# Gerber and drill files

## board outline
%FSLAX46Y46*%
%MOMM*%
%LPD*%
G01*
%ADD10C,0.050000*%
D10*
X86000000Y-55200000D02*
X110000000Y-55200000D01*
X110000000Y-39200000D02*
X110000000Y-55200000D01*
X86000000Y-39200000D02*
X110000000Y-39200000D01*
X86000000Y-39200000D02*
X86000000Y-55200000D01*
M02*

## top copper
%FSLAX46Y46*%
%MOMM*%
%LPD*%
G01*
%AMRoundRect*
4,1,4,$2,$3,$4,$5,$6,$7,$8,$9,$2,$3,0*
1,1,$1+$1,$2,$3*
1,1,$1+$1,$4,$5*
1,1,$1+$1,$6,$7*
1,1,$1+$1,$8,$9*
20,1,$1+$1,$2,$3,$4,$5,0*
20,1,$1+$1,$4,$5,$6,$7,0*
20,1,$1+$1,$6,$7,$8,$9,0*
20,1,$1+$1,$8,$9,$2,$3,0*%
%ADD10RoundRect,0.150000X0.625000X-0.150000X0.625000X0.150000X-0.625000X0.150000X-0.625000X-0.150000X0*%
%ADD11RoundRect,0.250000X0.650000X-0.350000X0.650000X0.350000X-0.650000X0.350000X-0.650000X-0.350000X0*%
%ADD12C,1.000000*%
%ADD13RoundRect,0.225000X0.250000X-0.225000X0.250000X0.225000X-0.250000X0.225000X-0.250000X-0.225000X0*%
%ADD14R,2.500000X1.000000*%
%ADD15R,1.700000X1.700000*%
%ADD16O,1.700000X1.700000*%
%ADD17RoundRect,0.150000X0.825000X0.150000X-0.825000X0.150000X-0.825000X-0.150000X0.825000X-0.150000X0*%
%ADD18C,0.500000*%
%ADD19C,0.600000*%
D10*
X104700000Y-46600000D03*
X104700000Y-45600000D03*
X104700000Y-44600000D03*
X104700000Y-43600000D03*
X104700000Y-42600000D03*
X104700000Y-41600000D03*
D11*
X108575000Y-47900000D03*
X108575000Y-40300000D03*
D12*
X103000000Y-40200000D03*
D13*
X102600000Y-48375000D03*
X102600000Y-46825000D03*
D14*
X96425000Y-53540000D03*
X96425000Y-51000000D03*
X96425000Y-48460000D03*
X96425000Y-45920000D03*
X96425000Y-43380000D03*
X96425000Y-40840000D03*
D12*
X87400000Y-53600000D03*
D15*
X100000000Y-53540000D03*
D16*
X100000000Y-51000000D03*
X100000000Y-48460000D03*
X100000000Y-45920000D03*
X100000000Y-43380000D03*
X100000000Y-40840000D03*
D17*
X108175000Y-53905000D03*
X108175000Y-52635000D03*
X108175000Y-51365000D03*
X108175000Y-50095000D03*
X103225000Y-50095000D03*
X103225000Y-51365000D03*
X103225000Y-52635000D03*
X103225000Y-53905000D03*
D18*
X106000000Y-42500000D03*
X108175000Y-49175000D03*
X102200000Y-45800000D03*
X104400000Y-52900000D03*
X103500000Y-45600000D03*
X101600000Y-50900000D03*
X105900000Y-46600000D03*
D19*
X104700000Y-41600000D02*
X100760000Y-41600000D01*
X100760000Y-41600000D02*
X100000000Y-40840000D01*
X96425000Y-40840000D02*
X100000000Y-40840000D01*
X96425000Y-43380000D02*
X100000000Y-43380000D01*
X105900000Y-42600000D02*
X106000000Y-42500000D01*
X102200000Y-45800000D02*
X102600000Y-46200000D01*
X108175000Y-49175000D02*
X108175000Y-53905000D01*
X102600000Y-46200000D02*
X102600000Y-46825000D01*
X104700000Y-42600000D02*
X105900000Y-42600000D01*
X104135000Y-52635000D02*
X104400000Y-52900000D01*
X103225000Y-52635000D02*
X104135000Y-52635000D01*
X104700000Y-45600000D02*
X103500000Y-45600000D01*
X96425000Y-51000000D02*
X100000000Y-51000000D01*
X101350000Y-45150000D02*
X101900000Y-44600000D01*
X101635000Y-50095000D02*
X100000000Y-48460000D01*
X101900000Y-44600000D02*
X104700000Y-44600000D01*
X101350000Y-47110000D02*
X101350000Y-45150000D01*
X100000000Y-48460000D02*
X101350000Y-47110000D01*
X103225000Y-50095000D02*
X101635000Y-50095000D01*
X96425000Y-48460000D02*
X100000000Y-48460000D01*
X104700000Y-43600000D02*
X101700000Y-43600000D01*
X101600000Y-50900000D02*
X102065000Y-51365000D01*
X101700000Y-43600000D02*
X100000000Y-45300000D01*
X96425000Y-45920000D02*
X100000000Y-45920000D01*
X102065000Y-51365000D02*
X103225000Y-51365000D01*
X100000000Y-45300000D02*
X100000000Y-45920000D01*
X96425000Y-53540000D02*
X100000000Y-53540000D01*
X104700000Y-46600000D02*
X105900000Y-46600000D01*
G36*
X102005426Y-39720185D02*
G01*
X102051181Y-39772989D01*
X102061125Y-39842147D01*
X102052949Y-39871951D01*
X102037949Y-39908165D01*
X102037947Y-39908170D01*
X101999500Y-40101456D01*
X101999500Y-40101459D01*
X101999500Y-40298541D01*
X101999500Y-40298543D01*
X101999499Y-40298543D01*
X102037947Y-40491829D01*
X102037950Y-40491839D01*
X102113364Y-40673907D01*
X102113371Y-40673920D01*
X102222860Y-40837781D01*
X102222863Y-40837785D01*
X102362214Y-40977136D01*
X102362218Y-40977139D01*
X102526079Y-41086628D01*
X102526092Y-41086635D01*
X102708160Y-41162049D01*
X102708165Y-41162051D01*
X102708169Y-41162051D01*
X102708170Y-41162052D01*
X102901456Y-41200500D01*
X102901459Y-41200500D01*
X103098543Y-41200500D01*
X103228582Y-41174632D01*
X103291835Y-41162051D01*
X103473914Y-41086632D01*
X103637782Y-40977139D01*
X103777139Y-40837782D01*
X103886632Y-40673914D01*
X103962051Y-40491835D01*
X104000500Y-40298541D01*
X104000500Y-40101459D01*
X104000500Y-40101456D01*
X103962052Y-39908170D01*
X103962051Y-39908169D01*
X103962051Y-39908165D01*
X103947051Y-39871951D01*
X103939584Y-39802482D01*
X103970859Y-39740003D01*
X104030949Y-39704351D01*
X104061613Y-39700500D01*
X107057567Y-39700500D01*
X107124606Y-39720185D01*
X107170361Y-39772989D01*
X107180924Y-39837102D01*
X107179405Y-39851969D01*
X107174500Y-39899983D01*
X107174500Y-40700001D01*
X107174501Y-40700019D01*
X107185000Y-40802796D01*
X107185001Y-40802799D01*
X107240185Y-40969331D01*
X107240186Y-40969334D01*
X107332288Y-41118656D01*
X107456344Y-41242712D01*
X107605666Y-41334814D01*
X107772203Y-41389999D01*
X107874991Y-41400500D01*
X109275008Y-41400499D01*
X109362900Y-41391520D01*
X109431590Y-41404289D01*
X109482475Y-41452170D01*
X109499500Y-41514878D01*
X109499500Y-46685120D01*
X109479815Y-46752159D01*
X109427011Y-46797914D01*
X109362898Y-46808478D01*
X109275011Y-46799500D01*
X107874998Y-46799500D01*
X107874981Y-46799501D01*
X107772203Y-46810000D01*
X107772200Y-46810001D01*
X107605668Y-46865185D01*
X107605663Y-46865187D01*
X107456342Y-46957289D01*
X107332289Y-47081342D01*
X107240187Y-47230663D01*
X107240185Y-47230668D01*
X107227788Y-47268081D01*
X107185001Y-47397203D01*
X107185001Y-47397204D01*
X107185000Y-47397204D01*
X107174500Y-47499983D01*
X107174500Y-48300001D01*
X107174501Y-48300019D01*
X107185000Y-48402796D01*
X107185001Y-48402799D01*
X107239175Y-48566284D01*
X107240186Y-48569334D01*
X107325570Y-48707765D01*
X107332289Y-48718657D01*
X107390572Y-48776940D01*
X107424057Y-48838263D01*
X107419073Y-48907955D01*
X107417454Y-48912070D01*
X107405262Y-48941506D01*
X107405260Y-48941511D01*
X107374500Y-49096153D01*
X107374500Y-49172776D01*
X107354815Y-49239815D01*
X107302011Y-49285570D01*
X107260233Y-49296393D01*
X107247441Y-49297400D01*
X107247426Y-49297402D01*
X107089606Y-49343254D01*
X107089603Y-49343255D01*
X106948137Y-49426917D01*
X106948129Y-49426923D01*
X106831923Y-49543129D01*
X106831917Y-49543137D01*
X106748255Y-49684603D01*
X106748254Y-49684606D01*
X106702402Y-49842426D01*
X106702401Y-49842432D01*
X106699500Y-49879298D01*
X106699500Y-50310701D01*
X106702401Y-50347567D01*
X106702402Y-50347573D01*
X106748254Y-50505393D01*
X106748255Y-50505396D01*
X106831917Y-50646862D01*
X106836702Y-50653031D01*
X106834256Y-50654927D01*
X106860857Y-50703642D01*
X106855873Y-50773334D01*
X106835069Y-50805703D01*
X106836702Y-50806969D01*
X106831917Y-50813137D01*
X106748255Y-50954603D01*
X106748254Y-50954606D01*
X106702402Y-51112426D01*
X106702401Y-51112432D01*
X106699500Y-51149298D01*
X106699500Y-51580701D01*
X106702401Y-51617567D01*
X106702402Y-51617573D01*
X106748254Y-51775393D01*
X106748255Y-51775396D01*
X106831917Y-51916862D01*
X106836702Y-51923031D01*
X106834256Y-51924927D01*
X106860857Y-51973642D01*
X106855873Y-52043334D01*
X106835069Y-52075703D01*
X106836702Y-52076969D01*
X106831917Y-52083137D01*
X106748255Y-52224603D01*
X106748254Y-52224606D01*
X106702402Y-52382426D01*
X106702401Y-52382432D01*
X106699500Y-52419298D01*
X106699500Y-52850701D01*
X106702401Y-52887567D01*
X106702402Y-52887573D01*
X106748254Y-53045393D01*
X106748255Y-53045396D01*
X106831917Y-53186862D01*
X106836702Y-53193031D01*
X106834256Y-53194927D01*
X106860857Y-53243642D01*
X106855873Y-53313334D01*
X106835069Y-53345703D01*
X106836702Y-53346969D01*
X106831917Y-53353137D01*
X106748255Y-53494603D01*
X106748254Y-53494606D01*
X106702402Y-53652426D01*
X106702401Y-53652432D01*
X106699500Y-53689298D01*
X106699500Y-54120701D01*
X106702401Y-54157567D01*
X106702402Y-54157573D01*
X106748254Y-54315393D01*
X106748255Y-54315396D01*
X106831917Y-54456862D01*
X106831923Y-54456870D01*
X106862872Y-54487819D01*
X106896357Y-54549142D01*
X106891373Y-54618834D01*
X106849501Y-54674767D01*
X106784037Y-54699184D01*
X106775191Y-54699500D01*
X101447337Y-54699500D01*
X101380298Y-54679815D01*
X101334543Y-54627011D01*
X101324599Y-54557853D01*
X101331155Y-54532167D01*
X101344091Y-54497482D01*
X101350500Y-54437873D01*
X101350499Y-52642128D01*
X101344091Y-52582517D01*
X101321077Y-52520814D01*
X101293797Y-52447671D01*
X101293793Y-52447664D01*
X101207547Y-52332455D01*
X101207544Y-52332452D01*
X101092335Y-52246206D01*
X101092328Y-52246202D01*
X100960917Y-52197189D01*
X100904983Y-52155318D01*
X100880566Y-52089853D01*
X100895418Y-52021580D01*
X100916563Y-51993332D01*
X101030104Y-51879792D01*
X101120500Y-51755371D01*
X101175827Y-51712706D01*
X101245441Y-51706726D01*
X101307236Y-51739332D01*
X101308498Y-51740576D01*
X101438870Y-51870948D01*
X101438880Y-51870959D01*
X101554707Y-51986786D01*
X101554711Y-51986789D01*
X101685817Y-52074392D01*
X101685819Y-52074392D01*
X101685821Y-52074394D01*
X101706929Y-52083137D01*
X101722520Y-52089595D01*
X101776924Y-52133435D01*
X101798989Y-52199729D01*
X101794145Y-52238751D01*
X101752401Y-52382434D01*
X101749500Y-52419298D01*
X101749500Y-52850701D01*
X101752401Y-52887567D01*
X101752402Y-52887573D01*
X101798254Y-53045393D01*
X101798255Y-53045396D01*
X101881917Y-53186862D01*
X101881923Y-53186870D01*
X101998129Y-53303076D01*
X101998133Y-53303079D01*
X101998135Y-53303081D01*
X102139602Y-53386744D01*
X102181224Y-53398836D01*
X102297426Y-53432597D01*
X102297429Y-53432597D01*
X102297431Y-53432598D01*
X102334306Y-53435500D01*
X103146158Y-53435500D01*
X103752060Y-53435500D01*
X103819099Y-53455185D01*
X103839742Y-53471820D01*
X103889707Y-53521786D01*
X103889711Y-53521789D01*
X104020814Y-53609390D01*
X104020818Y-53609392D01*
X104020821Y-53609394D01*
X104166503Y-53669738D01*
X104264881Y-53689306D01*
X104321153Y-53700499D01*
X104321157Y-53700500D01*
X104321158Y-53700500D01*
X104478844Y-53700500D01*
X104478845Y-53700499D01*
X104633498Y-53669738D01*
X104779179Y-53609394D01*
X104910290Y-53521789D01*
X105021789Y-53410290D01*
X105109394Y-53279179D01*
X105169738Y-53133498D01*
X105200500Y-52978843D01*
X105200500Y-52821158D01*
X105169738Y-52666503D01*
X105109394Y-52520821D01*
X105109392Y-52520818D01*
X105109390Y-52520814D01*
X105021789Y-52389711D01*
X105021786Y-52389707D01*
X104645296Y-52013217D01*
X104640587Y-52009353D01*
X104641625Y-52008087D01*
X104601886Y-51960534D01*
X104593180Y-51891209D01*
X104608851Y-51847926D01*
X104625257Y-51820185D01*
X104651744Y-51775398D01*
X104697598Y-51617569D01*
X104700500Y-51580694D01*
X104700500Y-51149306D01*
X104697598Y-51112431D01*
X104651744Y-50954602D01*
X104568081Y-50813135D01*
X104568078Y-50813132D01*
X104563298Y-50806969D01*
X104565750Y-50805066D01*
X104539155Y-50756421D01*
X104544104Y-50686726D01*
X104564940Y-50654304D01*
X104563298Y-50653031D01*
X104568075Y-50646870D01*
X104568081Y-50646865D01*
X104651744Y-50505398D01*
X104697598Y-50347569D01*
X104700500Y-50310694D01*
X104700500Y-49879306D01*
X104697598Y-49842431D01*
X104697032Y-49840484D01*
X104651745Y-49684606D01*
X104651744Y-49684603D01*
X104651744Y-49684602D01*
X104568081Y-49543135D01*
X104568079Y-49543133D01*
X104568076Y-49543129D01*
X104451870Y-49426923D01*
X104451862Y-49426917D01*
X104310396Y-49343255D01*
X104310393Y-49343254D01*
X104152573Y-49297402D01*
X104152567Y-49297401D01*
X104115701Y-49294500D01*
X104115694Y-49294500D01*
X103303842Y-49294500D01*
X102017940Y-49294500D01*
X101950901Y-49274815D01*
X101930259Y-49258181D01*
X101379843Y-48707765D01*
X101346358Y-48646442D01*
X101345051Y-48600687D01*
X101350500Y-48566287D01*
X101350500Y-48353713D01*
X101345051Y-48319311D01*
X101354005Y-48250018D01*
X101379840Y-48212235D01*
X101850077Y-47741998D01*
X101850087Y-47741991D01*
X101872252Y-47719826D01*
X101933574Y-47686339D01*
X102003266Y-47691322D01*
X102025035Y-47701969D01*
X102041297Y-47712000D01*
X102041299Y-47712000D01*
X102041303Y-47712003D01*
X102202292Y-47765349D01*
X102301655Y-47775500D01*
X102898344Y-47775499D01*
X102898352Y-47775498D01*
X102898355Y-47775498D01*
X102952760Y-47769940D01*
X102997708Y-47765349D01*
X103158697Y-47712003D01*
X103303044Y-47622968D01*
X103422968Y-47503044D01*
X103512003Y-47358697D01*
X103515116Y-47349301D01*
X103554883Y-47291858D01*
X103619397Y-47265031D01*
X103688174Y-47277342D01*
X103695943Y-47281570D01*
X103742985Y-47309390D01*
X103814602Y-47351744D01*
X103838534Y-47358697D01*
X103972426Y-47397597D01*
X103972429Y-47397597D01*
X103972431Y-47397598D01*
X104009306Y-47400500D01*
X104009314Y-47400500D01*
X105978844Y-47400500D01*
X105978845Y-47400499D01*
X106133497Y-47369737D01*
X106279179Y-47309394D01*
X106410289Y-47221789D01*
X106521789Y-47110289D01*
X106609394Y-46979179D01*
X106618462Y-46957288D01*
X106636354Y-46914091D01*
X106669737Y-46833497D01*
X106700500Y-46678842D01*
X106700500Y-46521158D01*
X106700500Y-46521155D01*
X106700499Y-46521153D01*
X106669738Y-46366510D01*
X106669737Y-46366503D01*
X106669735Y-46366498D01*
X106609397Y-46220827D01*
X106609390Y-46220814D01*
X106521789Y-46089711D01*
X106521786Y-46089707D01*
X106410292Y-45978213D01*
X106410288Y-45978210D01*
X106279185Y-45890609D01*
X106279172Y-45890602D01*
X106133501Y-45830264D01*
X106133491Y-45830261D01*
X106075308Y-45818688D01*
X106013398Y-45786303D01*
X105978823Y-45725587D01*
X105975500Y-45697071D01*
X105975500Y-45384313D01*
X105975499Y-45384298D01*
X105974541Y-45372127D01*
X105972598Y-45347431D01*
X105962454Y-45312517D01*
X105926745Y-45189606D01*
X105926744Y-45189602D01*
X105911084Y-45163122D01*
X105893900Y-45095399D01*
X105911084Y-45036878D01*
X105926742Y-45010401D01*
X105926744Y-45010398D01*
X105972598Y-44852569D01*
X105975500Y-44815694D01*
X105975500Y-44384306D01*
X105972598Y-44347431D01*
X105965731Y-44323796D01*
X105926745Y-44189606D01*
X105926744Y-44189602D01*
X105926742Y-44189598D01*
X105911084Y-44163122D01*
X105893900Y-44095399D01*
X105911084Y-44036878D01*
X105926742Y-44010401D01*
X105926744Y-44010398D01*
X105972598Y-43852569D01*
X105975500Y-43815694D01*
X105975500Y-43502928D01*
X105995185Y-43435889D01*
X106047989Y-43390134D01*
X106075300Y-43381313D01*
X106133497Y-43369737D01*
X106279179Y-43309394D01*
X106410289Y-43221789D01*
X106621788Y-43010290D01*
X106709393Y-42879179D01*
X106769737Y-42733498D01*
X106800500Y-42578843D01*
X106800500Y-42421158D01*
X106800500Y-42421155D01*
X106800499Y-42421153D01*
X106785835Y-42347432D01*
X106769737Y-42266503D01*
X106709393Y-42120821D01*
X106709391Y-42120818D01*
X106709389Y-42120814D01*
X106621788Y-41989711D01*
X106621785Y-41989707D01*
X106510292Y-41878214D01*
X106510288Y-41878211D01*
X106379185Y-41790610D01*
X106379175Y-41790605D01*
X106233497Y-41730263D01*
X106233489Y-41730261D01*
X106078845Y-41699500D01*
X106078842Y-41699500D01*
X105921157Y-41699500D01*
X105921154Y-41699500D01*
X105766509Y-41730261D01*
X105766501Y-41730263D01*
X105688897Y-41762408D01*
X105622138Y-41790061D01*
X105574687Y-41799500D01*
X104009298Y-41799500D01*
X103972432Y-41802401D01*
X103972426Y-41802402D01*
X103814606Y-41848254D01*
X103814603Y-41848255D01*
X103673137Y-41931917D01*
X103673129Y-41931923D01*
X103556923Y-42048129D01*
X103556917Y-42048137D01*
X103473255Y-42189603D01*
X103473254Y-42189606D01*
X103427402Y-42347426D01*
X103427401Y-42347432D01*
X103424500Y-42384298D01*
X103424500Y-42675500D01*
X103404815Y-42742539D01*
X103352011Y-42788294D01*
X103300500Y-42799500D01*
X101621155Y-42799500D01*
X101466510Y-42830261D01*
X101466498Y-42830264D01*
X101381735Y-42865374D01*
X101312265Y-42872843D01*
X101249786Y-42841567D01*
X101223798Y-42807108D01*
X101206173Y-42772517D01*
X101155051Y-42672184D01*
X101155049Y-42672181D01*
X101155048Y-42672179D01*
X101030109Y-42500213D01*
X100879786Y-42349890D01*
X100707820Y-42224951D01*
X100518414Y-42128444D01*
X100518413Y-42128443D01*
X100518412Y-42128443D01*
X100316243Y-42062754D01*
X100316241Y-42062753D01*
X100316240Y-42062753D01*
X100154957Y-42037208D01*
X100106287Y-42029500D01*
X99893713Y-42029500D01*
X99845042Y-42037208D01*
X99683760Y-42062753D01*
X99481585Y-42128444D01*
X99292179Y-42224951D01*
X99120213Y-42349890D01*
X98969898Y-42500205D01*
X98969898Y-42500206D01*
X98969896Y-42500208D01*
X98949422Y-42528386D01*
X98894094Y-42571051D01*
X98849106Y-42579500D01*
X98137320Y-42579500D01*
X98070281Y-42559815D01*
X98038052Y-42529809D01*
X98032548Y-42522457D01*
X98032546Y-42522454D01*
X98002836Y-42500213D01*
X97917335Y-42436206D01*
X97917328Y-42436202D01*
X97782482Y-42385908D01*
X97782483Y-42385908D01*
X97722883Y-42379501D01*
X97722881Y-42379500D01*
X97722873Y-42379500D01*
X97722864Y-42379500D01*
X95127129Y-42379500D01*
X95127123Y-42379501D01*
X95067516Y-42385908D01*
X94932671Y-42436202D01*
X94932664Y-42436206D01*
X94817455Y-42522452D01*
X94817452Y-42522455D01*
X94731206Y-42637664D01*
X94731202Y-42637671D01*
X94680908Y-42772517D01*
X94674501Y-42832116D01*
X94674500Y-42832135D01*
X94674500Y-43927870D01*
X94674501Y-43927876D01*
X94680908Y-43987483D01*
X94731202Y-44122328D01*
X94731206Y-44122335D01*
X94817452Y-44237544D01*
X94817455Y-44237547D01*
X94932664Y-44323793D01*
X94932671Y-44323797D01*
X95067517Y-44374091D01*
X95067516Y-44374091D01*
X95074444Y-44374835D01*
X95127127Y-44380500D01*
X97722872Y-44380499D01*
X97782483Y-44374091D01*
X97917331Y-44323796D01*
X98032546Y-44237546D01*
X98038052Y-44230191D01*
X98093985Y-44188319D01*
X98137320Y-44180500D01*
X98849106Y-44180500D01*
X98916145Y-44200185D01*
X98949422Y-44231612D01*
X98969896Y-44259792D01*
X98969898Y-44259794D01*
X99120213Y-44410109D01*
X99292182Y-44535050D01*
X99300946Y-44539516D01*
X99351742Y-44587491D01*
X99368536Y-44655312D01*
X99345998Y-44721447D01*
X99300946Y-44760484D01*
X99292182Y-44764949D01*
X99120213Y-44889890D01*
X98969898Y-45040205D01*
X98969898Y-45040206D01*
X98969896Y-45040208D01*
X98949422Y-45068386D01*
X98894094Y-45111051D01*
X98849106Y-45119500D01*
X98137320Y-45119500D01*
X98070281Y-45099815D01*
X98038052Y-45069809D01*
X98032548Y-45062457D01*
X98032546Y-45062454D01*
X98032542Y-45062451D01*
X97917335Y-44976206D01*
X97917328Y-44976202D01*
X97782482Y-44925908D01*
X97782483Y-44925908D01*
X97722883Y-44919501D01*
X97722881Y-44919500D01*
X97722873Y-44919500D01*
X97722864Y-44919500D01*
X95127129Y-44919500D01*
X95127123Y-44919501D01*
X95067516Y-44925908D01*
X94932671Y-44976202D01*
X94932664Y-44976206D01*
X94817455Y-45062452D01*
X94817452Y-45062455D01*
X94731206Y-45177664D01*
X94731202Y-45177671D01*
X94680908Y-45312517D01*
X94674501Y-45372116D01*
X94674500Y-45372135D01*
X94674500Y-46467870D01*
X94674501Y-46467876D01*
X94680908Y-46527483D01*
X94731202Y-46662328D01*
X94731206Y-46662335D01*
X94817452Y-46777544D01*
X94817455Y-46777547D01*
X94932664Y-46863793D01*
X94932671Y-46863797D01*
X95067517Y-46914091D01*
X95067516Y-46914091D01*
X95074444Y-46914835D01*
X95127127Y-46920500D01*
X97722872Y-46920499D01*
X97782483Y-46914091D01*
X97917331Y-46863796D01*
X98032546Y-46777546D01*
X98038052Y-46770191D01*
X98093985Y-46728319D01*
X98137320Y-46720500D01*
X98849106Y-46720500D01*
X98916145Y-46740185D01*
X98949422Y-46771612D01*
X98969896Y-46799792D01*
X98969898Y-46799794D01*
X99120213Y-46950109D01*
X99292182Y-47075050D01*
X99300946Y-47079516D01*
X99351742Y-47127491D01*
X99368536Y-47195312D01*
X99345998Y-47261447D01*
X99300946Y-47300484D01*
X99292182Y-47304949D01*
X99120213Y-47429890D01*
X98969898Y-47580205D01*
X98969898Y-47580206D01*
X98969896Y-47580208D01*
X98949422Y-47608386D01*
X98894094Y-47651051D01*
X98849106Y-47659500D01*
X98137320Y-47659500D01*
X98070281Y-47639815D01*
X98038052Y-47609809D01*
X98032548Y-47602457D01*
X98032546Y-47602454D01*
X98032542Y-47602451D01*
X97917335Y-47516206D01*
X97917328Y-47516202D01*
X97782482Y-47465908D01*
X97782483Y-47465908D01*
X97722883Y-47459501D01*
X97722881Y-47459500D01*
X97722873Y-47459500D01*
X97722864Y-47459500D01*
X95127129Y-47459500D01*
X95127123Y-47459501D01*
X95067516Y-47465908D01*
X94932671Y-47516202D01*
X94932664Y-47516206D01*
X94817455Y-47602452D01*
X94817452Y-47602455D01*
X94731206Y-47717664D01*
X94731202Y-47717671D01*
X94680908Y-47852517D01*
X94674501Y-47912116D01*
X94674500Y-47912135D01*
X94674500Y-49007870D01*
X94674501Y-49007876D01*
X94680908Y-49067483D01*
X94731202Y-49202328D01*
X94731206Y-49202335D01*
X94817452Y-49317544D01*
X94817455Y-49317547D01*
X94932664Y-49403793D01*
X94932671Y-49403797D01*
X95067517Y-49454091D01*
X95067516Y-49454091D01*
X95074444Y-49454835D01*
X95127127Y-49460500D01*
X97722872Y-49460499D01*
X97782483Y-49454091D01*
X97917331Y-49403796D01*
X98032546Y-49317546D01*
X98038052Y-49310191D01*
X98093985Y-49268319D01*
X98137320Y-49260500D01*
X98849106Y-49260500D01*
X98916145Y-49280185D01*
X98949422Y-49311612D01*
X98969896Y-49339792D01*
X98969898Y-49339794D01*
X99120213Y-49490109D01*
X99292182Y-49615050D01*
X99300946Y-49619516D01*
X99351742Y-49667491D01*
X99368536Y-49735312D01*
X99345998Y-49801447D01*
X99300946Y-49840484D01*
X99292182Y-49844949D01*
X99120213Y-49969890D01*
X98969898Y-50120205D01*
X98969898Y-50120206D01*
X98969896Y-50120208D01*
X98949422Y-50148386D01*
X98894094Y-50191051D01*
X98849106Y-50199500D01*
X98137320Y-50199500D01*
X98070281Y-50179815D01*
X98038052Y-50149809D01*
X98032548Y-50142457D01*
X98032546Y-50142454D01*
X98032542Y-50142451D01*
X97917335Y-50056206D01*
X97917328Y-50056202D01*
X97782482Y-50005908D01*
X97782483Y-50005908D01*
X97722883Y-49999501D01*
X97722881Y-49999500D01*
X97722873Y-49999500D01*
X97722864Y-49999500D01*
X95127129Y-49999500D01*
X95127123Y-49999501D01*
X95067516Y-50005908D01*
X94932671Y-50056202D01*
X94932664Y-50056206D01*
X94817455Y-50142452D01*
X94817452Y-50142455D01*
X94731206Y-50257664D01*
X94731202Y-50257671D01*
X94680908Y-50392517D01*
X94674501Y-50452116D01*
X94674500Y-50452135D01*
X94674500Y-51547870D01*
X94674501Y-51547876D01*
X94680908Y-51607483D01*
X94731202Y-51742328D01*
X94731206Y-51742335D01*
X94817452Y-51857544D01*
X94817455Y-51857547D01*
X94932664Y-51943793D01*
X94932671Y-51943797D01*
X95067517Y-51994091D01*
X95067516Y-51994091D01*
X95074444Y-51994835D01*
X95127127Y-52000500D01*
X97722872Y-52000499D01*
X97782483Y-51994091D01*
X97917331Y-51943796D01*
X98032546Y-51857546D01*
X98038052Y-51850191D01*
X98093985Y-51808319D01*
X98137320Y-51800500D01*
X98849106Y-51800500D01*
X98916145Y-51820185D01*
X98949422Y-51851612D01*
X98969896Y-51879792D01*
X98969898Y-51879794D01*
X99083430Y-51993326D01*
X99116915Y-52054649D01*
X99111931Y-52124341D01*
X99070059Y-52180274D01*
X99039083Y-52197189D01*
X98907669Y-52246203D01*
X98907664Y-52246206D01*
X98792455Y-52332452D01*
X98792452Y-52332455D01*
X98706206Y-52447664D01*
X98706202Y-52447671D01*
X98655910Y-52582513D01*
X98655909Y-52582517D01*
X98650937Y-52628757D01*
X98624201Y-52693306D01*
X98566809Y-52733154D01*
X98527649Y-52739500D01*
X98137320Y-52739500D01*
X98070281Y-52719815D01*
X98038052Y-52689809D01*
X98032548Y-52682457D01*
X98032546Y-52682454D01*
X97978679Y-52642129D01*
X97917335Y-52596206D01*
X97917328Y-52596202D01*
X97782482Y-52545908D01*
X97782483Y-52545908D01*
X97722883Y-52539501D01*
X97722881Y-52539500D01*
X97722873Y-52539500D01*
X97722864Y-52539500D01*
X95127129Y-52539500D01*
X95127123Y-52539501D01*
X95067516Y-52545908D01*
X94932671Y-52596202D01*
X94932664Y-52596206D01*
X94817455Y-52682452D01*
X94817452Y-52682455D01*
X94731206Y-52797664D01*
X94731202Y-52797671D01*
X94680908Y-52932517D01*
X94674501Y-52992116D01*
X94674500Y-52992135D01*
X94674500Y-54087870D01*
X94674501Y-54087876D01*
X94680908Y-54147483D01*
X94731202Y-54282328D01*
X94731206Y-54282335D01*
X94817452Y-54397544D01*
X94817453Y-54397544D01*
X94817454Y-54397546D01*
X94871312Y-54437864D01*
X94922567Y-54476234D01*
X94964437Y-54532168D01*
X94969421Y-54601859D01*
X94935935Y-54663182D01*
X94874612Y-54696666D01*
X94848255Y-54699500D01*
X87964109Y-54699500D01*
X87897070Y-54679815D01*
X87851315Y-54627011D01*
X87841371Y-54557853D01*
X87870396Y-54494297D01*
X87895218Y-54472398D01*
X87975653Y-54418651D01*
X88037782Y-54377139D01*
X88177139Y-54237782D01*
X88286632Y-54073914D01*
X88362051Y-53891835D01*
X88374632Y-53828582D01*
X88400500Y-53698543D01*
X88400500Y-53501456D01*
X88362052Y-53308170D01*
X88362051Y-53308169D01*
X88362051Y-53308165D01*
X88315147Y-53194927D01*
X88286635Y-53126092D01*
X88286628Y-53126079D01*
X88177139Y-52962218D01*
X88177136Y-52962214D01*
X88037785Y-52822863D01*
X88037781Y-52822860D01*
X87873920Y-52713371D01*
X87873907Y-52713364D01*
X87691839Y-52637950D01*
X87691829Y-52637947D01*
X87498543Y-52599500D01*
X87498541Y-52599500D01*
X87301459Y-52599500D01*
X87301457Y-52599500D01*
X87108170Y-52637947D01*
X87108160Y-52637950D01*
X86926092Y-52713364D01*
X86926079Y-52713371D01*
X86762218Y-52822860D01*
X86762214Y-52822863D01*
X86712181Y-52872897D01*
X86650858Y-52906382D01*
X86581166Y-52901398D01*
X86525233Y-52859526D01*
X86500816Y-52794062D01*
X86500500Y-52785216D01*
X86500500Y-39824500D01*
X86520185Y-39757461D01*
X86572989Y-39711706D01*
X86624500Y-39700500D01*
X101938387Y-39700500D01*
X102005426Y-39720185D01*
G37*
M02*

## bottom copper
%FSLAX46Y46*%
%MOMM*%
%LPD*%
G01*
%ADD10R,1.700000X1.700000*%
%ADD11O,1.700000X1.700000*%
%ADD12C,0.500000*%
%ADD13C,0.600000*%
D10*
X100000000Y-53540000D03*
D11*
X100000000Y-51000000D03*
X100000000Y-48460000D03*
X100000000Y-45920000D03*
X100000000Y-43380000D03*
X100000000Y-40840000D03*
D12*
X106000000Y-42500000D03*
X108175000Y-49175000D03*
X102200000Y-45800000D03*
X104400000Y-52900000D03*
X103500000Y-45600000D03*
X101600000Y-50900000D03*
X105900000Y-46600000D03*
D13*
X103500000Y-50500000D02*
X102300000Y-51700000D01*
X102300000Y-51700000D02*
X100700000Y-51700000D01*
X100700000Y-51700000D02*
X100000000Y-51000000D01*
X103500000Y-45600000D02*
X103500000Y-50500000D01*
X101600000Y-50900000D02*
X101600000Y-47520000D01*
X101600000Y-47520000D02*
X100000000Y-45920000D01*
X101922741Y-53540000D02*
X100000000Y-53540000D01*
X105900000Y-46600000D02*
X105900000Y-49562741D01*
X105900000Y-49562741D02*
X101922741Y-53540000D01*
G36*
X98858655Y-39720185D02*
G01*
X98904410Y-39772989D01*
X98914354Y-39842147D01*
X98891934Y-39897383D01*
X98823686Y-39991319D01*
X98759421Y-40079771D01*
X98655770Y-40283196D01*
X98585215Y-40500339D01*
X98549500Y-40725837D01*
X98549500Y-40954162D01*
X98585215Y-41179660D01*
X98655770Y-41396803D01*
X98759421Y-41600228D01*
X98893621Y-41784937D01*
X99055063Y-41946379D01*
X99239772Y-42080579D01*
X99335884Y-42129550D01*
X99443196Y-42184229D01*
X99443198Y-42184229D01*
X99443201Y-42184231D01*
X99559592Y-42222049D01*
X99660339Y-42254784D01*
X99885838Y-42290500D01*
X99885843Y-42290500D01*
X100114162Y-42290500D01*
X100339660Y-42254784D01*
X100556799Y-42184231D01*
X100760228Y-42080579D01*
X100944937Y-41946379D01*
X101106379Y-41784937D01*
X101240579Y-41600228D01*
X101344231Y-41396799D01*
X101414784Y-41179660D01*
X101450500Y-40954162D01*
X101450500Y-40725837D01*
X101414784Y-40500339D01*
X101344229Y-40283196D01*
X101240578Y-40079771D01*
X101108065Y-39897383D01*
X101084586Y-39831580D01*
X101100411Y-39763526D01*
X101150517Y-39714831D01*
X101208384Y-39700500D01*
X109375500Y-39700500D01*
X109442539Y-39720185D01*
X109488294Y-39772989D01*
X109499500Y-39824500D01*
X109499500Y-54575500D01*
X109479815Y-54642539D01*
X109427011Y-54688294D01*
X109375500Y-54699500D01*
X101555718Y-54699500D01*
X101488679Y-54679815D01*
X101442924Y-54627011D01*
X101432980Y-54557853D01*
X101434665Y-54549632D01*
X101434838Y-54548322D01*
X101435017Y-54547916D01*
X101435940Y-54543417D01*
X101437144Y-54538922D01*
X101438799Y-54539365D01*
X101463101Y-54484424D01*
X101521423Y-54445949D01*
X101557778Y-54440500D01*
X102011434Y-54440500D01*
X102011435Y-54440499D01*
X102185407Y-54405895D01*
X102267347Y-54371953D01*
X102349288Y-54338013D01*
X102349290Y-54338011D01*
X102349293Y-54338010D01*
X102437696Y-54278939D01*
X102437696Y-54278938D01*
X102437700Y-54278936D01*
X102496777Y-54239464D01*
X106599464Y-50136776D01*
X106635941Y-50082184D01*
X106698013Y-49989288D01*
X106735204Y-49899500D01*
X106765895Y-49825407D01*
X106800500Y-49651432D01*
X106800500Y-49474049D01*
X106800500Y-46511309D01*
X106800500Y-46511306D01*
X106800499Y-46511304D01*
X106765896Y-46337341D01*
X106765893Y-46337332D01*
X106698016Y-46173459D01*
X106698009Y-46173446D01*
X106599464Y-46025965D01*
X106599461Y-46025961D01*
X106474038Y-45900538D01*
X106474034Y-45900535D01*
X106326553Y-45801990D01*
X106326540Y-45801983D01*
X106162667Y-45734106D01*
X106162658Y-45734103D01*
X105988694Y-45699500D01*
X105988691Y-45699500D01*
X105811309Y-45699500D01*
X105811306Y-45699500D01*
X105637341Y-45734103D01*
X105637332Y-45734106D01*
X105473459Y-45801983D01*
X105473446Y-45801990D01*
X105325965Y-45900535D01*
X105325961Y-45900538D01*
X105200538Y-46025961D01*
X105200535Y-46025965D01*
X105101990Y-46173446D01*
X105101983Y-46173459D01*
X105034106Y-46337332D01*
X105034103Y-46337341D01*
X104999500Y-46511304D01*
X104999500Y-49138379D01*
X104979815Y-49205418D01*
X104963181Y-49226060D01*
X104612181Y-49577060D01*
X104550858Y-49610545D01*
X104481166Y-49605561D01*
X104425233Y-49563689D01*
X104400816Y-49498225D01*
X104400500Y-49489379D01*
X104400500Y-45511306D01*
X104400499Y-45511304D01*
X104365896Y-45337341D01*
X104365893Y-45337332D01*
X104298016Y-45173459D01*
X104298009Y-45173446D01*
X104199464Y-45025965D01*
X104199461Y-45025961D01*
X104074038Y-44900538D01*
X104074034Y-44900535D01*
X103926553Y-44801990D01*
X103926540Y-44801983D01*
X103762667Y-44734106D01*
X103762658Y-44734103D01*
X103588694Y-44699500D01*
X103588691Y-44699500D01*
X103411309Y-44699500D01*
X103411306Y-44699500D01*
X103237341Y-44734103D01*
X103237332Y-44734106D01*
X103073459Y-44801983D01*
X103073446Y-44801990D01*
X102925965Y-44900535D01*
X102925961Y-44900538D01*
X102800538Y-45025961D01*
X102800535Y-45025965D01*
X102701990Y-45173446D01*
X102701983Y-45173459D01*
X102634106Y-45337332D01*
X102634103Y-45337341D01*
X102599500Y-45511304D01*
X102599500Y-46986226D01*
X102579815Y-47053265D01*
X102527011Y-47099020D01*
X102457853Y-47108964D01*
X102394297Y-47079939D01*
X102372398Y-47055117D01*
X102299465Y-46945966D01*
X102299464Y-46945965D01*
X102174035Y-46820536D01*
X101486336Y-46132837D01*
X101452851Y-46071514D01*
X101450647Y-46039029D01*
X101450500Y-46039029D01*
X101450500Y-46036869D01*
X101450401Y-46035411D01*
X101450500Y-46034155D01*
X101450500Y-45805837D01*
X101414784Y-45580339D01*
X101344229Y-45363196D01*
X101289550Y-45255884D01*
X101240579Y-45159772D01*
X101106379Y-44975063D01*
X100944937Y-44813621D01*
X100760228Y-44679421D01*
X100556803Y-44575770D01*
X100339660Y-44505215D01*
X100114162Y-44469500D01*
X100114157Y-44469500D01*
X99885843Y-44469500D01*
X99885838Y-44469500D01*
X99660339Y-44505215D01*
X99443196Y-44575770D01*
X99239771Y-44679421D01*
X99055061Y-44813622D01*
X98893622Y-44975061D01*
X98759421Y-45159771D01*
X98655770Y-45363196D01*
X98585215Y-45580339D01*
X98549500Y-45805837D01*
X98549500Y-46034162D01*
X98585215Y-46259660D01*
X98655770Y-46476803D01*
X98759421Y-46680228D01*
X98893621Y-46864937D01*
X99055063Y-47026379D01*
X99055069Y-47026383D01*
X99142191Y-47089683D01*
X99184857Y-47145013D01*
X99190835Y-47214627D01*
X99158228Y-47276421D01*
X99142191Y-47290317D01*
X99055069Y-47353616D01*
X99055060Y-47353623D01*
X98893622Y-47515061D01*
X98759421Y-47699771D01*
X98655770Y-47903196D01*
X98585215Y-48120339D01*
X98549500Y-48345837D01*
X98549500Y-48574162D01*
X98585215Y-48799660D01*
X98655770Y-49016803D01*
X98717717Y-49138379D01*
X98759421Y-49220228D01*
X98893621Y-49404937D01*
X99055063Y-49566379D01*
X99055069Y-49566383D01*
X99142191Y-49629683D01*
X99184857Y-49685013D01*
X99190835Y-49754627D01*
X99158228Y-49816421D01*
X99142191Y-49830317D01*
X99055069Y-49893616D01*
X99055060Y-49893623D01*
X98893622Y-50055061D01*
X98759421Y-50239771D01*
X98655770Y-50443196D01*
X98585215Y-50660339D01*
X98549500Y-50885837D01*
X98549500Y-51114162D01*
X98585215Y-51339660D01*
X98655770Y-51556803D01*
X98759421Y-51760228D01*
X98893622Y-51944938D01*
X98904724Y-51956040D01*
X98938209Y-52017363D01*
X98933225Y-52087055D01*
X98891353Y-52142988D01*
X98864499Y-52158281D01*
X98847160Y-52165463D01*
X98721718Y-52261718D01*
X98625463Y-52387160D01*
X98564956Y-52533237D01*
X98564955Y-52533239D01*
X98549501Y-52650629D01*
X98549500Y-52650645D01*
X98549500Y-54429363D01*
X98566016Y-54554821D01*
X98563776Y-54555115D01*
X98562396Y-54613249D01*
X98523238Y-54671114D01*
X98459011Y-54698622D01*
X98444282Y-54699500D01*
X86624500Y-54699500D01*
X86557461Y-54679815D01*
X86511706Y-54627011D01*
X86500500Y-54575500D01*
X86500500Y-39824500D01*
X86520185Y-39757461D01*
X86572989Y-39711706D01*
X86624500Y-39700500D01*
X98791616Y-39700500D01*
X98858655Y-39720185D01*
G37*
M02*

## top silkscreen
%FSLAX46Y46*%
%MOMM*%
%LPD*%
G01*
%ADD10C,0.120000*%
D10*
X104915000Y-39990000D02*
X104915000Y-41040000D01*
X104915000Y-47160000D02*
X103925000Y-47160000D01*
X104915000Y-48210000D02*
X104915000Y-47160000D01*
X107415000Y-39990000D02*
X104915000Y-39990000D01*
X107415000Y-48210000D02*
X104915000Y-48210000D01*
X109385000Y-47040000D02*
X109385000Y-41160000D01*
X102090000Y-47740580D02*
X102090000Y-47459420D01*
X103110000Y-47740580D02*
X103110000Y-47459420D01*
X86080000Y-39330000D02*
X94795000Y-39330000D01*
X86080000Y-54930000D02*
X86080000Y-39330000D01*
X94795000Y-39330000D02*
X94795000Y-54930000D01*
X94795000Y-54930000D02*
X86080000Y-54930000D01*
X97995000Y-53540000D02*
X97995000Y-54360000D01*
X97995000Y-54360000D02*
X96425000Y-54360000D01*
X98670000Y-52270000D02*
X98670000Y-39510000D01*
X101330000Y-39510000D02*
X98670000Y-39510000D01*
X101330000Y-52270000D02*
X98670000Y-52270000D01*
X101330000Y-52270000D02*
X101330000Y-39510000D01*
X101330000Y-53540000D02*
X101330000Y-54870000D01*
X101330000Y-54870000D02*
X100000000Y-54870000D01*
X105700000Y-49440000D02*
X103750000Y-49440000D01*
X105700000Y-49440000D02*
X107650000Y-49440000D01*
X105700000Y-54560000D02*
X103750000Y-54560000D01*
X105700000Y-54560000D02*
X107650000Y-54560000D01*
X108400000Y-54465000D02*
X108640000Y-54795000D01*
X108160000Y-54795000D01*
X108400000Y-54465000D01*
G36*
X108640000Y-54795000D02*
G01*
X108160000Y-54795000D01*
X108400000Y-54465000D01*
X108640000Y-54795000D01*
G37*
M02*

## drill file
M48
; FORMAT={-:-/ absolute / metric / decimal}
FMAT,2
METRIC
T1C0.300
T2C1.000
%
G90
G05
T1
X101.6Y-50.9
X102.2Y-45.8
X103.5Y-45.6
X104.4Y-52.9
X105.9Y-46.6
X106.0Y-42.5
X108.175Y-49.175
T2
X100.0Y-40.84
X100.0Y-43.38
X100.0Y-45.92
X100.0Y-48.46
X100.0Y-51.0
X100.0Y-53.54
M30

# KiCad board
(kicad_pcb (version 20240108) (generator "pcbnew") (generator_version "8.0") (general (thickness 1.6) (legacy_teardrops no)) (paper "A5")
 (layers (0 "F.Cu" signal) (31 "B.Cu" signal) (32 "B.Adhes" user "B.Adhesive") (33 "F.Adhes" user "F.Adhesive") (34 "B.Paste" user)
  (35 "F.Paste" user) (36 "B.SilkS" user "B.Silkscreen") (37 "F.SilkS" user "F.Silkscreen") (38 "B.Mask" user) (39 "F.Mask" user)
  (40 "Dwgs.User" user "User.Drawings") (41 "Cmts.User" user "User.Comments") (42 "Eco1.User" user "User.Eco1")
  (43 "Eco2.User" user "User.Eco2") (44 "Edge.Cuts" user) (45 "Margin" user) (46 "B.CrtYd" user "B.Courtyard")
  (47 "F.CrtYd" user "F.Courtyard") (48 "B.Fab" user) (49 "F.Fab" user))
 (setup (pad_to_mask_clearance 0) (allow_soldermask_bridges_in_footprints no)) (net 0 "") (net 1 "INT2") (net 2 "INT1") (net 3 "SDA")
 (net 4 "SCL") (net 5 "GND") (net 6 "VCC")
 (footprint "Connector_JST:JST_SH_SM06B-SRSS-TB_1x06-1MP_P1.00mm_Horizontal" (layer "F.Cu") (at 106.7 44.1 90)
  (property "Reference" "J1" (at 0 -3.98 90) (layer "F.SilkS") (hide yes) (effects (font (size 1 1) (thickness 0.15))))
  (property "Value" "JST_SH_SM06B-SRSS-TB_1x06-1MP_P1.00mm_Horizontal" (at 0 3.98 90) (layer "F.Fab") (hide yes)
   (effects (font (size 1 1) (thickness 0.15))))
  (fp_line (start 4.11 -1.785) (end 3.06 -1.785) (stroke (width 0.12) (type solid)) (layer "F.SilkS"))
  (fp_line (start -3.06 -1.785) (end -3.06 -2.775) (stroke (width 0.12) (type solid)) (layer "F.SilkS"))
  (fp_line (start -4.11 -1.785) (end -3.06 -1.785) (stroke (width 0.12) (type solid)) (layer "F.SilkS"))
  (fp_line (start 4.11 0.715) (end 4.11 -1.785) (stroke (width 0.12) (type solid)) (layer "F.SilkS"))
  (fp_line (start -4.11 0.715) (end -4.11 -1.785) (stroke (width 0.12) (type solid)) (layer "F.SilkS"))
  (fp_line (start -2.94 2.685) (end 2.94 2.685) (stroke (width 0.12) (type solid)) (layer "F.SilkS"))
  (pad "1" smd roundrect (at -2.5 -2 90) (size 0.6 1.55) (layers "F.Cu" "F.Paste" "F.Mask") (roundrect_rratio 0.25) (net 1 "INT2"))
  (pad "2" smd roundrect (at -1.5 -2 90) (size 0.6 1.55) (layers "F.Cu" "F.Paste" "F.Mask") (roundrect_rratio 0.25) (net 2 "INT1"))
  (pad "3" smd roundrect (at -0.5 -2 90) (size 0.6 1.55) (layers "F.Cu" "F.Paste" "F.Mask") (roundrect_rratio 0.25) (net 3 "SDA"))
  (pad "4" smd roundrect (at 0.5 -2 90) (size 0.6 1.55) (layers "F.Cu" "F.Paste" "F.Mask") (roundrect_rratio 0.25) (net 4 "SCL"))
  (pad "5" smd roundrect (at 1.5 -2 90) (size 0.6 1.55) (layers "F.Cu" "F.Paste" "F.Mask") (roundrect_rratio 0.25) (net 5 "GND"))
  (pad "6" smd roundrect (at 2.5 -2 90) (size 0.6 1.55) (layers "F.Cu" "F.Paste" "F.Mask") (roundrect_rratio 0.25) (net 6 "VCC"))
  (pad "MP" smd roundrect (at -3.8 1.875 90) (size 1.2 1.8) (layers "F.Cu" "F.Paste" "F.Mask") (roundrect_rratio 0.208333))
  (pad "MP" smd roundrect (at 3.8 1.875 90) (size 1.2 1.8) (layers "F.Cu" "F.Paste" "F.Mask") (roundrect_rratio 0.208333)))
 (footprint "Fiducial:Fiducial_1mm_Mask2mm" (layer "F.Cu") (at 103 40.2)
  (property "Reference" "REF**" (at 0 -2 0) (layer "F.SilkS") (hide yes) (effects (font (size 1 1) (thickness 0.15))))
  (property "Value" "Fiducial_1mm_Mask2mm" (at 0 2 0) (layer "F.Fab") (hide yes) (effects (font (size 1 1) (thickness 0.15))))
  (pad "" smd circle (at 0 0) (size 1 1) (layers "F.Cu" "F.Mask") (solder_mask_margin 0.5) (clearance 0.5)))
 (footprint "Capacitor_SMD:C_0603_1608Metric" (layer "F.Cu") (at 102.6 47.6 90)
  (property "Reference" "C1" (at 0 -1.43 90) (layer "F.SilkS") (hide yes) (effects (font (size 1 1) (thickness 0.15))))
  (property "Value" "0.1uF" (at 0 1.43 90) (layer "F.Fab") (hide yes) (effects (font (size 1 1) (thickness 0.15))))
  (fp_line (start -0.14058 -0.51) (end 0.14058 -0.51) (stroke (width 0.12) (type solid)) (layer "F.SilkS"))
  (fp_line (start -0.14058 0.51) (end 0.14058 0.51) (stroke (width 0.12) (type solid)) (layer "F.SilkS"))
  (pad "1" smd roundrect (at -0.775 0 90) (size 0.9 0.95) (layers "F.Cu" "F.Paste" "F.Mask") (roundrect_rratio 0.25) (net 6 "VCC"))
  (pad "2" smd roundrect (at 0.775 0 90) (size 0.9 0.95) (layers "F.Cu" "F.Paste" "F.Mask") (roundrect_rratio 0.25) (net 5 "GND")))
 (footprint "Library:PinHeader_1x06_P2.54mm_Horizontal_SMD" (layer "F.Cu") (at 90.9 51 180)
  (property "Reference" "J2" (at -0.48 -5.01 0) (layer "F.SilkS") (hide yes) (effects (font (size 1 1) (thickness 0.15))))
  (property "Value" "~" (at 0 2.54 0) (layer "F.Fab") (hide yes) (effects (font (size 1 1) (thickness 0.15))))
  (fp_line (start 4.82 11.67) (end -3.895 11.67) (stroke (width 0.12) (type solid)) (layer "F.SilkS"))
  (fp_line (start 4.82 -3.93) (end 4.82 11.67) (stroke (width 0.12) (type solid)) (layer "F.SilkS"))
  (fp_line (start -3.895 11.67) (end -3.895 -3.93) (stroke (width 0.12) (type solid)) (layer "F.SilkS"))
  (fp_line (start -3.895 -3.93) (end 4.82 -3.93) (stroke (width 0.12) (type solid)) (layer "F.SilkS"))
  (fp_line (start -7.095 -2.54) (end -7.095 -3.36) (stroke (width 0.12) (type solid)) (layer "F.SilkS"))
  (fp_line (start -7.095 -3.36) (end -5.525 -3.36) (stroke (width 0.12) (type solid)) (layer "F.SilkS"))
  (pad "1" smd rect (at -5.525 -2.54 180) (size 2.5 1) (layers "F.Cu" "F.Paste" "F.Mask") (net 1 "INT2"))
  (pad "2" smd rect (at -5.525 0 180) (size 2.5 1) (layers "F.Cu" "F.Paste" "F.Mask") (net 2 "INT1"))
  (pad "3" smd rect (at -5.525 2.54 180) (size 2.5 1) (layers "F.Cu" "F.Paste" "F.Mask") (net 3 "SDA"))
  (pad "4" smd rect (at -5.525 5.08 180) (size 2.5 1) (layers "F.Cu" "F.Paste" "F.Mask") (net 4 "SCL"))
  (pad "5" smd rect (at -5.525 7.62 180) (size 2.5 1) (layers "F.Cu" "F.Paste" "F.Mask") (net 5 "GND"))
  (pad "6" smd rect (at -5.525 10.16 180) (size 2.5 1) (layers "F.Cu" "F.Paste" "F.Mask") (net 6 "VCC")))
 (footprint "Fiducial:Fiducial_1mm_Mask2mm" (layer "F.Cu") (at 87.4 53.6)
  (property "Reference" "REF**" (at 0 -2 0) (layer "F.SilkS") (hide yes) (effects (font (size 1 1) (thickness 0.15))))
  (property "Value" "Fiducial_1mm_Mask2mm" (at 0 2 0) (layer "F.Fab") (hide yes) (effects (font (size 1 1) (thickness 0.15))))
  (pad "" smd circle (at 0 0) (size 1 1) (layers "F.Cu" "F.Mask") (solder_mask_margin 0.5) (clearance 0.5)))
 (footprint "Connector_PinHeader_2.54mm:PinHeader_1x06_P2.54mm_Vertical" (layer "F.Cu") (at 100 53.54 180)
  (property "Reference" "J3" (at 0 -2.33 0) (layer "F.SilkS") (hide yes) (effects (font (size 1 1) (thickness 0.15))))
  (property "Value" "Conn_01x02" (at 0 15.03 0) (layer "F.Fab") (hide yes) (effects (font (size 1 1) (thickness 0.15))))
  (fp_line (start 1.33 1.27) (end 1.33 14.03) (stroke (width 0.12) (type solid)) (layer "F.SilkS"))
  (fp_line (start -1.33 14.03) (end 1.33 14.03) (stroke (width 0.12) (type solid)) (layer "F.SilkS"))
  (fp_line (start -1.33 1.27) (end 1.33 1.27) (stroke (width 0.12) (type solid)) (layer "F.SilkS"))
  (fp_line (start -1.33 1.27) (end -1.33 14.03) (stroke (width 0.12) (type solid)) (layer "F.SilkS"))
  (fp_line (start -1.33 0) (end -1.33 -1.33) (stroke (width 0.12) (type solid)) (layer "F.SilkS"))
  (fp_line (start -1.33 -1.33) (end 0 -1.33) (stroke (width 0.12) (type solid)) (layer "F.SilkS"))
  (pad "1" thru_hole rect (at 0 0 180) (size 1.7 1.7) (drill 1) (layers "*.Cu" "*.Mask") (remove_unused_layers no) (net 1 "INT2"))
  (pad "2" thru_hole oval (at 0 2.54 180) (size 1.7 1.7) (drill 1) (layers "*.Cu" "*.Mask") (remove_unused_layers no) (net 2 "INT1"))
  (pad "3" thru_hole oval (at 0 5.08 180) (size 1.7 1.7) (drill 1) (layers "*.Cu" "*.Mask") (remove_unused_layers no) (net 3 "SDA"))
  (pad "4" thru_hole oval (at 0 7.62 180) (size 1.7 1.7) (drill 1) (layers "*.Cu" "*.Mask") (remove_unused_layers no) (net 4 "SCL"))
  (pad "5" thru_hole oval (at 0 10.16 180) (size 1.7 1.7) (drill 1) (layers "*.Cu" "*.Mask") (remove_unused_layers no) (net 5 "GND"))
  (pad "6" thru_hole oval (at 0 12.7 180) (size 1.7 1.7) (drill 1) (layers "*.Cu" "*.Mask") (remove_unused_layers no) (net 6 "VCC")))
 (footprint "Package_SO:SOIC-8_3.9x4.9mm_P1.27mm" (layer "F.Cu") (at 105.7 52 180)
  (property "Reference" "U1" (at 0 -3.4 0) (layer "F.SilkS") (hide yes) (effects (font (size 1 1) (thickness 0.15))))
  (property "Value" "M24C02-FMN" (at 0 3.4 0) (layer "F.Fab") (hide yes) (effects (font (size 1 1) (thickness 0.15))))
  (fp_line (start 0 2.56) (end 1.95 2.56) (stroke (width 0.12) (type solid)) (layer "F.SilkS"))
  (fp_line (start 0 2.56) (end -1.95 2.56) (stroke (width 0.12) (type solid)) (layer "F.SilkS"))
  (fp_line (start 0 -2.56) (end 1.95 -2.56) (stroke (width 0.12) (type solid)) (layer "F.SilkS"))
  (fp_line (start 0 -2.56) (end -1.95 -2.56) (stroke (width 0.12) (type solid)) (layer "F.SilkS"))
  (fp_poly
   (pts (xy -2.7 -2.465) (xy -2.94 -2.795) (xy -2.46 -2.795) (xy -2.7 -2.465)) (stroke (width 0.12) (type solid)) (fill solid)
   (layer "F.SilkS"))
  (pad "1" smd roundrect (at -2.475 -1.905 180) (size 1.95 0.6) (layers "F.Cu" "F.Paste" "F.Mask") (roundrect_rratio 0.25) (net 5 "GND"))
  (pad "2" smd roundrect (at -2.475 -0.635 180) (size 1.95 0.6) (layers "F.Cu" "F.Paste" "F.Mask") (roundrect_rratio 0.25) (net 5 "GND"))
  (pad "3" smd roundrect (at -2.475 0.635 180) (size 1.95 0.6) (layers "F.Cu" "F.Paste" "F.Mask") (roundrect_rratio 0.25) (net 5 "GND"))
  (pad "4" smd roundrect (at -2.475 1.905 180) (size 1.95 0.6) (layers "F.Cu" "F.Paste" "F.Mask") (roundrect_rratio 0.25) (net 5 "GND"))
  (pad "5" smd roundrect (at 2.475 1.905 180) (size 1.95 0.6) (layers "F.Cu" "F.Paste" "F.Mask") (roundrect_rratio 0.25) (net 3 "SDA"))
  (pad "6" smd roundrect (at 2.475 0.635 180) (size 1.95 0.6) (layers "F.Cu" "F.Paste" "F.Mask") (roundrect_rratio 0.25) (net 4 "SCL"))
  (pad "7" smd roundrect (at 2.475 -0.635 180) (size 1.95 0.6) (layers "F.Cu" "F.Paste" "F.Mask") (roundrect_rratio 0.25) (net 5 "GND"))
  (pad "8" smd roundrect (at 2.475 -1.905 180) (size 1.95 0.6) (layers "F.Cu" "F.Paste" "F.Mask") (roundrect_rratio 0.25) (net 6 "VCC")))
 (gr_line (start 86 55.2) (end 110 55.2) (stroke (width 0.05) (type default)) (layer "Edge.Cuts"))
 (gr_line (start 110 39.2) (end 110 55.2) (stroke (width 0.05) (type default)) (layer "Edge.Cuts"))
 (gr_line (start 86 39.2) (end 110 39.2) (stroke (width 0.05) (type default)) (layer "Edge.Cuts"))
 (gr_line (start 86 39.2) (end 86 55.2) (stroke (width 0.05) (type default)) (layer "Edge.Cuts"))
 (segment (start 104.7 41.6) (end 100.76 41.6) (width 0.6) (layer "F.Cu") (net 6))
 (segment (start 100.76 41.6) (end 100 40.84) (width 0.6) (layer "F.Cu") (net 6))
 (segment (start 96.425 40.84) (end 100 40.84) (width 0.6) (layer "F.Cu") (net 6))
 (segment (start 96.425 43.38) (end 100 43.38) (width 0.6) (layer "F.Cu") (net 5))
 (segment (start 105.9 42.6) (end 106 42.5) (width 0.6) (layer "F.Cu") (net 5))
 (segment (start 102.2 45.8) (end 102.6 46.2) (width 0.6) (layer "F.Cu") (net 5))
 (segment (start 108.175 49.175) (end 108.175 53.905) (width 0.6) (layer "F.Cu") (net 5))
 (segment (start 102.6 46.2) (end 102.6 46.825) (width 0.6) (layer "F.Cu") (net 5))
 (segment (start 104.7 42.6) (end 105.9 42.6) (width 0.6) (layer "F.Cu") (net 5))
 (segment (start 104.135 52.635) (end 104.4 52.9) (width 0.6) (layer "F.Cu") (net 5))
 (segment (start 103.225 52.635) (end 104.135 52.635) (width 0.6) (layer "F.Cu") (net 5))
 (via (at 106 42.5) (size 0.5) (drill 0.3) (layers "F.Cu" "B.Cu") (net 5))
 (via (at 108.175 49.175) (size 0.5) (drill 0.3) (layers "F.Cu" "B.Cu") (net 5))
 (via (at 102.2 45.8) (size 0.5) (drill 0.3) (layers "F.Cu" "B.Cu") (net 5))
 (via (at 104.4 52.9) (size 0.5) (drill 0.3) (layers "F.Cu" "B.Cu") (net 5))
 (segment (start 104.7 45.6) (end 103.5 45.6) (width 0.6) (layer "F.Cu") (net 2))
 (segment (start 96.425 51) (end 100 51) (width 0.6) (layer "F.Cu") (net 2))
 (via (at 103.5 45.6) (size 0.5) (drill 0.3) (layers "F.Cu" "B.Cu") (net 2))
 (segment (start 103.5 50.5) (end 102.3 51.7) (width 0.6) (layer "B.Cu") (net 2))
 (segment (start 102.3 51.7) (end 100.7 51.7) (width 0.6) (layer "B.Cu") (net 2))
 (segment (start 100.7 51.7) (end 100 51) (width 0.6) (layer "B.Cu") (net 2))
 (segment (start 103.5 45.6) (end 103.5 50.5) (width 0.6) (layer "B.Cu") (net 2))
 (segment (start 101.35 45.15) (end 101.9 44.6) (width 0.6) (layer "F.Cu") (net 3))
 (segment (start 101.635 50.095) (end 100 48.46) (width 0.6) (layer "F.Cu") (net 3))
 (segment (start 101.9 44.6) (end 104.7 44.6) (width 0.6) (layer "F.Cu") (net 3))
 (segment (start 101.35 47.11) (end 101.35 45.15) (width 0.6) (layer "F.Cu") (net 3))
 (segment (start 100 48.46) (end 101.35 47.11) (width 0.6) (layer "F.Cu") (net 3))
 (segment (start 103.225 50.095) (end 101.635 50.095) (width 0.6) (layer "F.Cu") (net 3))
 (segment (start 96.425 48.46) (end 100 48.46) (width 0.6) (layer "F.Cu") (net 3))
 (segment (start 104.7 43.6) (end 101.7 43.6) (width 0.6) (layer "F.Cu") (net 4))
 (segment (start 101.6 50.9) (end 102.065 51.365) (width 0.6) (layer "F.Cu") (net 4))
 (segment (start 101.7 43.6) (end 100 45.3) (width 0.6) (layer "F.Cu") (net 4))
 (segment (start 96.425 45.92) (end 100 45.92) (width 0.6) (layer "F.Cu") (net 4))
 (segment (start 102.065 51.365) (end 103.225 51.365) (width 0.6) (layer "F.Cu") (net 4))
 (segment (start 100 45.3) (end 100 45.92) (width 0.6) (layer "F.Cu") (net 4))
 (via (at 101.6 50.9) (size 0.5) (drill 0.3) (layers "F.Cu" "B.Cu") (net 4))
 (segment (start 101.6 50.9) (end 101.6 47.52) (width 0.6) (layer "B.Cu") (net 4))
 (segment (start 101.6 47.52) (end 100 45.92) (width 0.6) (layer "B.Cu") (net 4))
 (segment (start 96.425 53.54) (end 100 53.54) (width 0.6) (layer "F.Cu") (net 1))
 (segment (start 104.7 46.6) (end 105.9 46.6) (width 0.6) (layer "F.Cu") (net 1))
 (via (at 105.9 46.6) (size 0.5) (drill 0.3) (layers "F.Cu" "B.Cu") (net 1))
 (segment (start 101.922741 53.54) (end 100 53.54) (width 0.6) (layer "B.Cu") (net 1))
 (segment (start 105.9 46.6) (end 105.9 49.562741) (width 0.6) (layer "B.Cu") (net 1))
 (segment (start 105.9 49.562741) (end 101.922741 53.54) (width 0.6) (layer "B.Cu") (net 1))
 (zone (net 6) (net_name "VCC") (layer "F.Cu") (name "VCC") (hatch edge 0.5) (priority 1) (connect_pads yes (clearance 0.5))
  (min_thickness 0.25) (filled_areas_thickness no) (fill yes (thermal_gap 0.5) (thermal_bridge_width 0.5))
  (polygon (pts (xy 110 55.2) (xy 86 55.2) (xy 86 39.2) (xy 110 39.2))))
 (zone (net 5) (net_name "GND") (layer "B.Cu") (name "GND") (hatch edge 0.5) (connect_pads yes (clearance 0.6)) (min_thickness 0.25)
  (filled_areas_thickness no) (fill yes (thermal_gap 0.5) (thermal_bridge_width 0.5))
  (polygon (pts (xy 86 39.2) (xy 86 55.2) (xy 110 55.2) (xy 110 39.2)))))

